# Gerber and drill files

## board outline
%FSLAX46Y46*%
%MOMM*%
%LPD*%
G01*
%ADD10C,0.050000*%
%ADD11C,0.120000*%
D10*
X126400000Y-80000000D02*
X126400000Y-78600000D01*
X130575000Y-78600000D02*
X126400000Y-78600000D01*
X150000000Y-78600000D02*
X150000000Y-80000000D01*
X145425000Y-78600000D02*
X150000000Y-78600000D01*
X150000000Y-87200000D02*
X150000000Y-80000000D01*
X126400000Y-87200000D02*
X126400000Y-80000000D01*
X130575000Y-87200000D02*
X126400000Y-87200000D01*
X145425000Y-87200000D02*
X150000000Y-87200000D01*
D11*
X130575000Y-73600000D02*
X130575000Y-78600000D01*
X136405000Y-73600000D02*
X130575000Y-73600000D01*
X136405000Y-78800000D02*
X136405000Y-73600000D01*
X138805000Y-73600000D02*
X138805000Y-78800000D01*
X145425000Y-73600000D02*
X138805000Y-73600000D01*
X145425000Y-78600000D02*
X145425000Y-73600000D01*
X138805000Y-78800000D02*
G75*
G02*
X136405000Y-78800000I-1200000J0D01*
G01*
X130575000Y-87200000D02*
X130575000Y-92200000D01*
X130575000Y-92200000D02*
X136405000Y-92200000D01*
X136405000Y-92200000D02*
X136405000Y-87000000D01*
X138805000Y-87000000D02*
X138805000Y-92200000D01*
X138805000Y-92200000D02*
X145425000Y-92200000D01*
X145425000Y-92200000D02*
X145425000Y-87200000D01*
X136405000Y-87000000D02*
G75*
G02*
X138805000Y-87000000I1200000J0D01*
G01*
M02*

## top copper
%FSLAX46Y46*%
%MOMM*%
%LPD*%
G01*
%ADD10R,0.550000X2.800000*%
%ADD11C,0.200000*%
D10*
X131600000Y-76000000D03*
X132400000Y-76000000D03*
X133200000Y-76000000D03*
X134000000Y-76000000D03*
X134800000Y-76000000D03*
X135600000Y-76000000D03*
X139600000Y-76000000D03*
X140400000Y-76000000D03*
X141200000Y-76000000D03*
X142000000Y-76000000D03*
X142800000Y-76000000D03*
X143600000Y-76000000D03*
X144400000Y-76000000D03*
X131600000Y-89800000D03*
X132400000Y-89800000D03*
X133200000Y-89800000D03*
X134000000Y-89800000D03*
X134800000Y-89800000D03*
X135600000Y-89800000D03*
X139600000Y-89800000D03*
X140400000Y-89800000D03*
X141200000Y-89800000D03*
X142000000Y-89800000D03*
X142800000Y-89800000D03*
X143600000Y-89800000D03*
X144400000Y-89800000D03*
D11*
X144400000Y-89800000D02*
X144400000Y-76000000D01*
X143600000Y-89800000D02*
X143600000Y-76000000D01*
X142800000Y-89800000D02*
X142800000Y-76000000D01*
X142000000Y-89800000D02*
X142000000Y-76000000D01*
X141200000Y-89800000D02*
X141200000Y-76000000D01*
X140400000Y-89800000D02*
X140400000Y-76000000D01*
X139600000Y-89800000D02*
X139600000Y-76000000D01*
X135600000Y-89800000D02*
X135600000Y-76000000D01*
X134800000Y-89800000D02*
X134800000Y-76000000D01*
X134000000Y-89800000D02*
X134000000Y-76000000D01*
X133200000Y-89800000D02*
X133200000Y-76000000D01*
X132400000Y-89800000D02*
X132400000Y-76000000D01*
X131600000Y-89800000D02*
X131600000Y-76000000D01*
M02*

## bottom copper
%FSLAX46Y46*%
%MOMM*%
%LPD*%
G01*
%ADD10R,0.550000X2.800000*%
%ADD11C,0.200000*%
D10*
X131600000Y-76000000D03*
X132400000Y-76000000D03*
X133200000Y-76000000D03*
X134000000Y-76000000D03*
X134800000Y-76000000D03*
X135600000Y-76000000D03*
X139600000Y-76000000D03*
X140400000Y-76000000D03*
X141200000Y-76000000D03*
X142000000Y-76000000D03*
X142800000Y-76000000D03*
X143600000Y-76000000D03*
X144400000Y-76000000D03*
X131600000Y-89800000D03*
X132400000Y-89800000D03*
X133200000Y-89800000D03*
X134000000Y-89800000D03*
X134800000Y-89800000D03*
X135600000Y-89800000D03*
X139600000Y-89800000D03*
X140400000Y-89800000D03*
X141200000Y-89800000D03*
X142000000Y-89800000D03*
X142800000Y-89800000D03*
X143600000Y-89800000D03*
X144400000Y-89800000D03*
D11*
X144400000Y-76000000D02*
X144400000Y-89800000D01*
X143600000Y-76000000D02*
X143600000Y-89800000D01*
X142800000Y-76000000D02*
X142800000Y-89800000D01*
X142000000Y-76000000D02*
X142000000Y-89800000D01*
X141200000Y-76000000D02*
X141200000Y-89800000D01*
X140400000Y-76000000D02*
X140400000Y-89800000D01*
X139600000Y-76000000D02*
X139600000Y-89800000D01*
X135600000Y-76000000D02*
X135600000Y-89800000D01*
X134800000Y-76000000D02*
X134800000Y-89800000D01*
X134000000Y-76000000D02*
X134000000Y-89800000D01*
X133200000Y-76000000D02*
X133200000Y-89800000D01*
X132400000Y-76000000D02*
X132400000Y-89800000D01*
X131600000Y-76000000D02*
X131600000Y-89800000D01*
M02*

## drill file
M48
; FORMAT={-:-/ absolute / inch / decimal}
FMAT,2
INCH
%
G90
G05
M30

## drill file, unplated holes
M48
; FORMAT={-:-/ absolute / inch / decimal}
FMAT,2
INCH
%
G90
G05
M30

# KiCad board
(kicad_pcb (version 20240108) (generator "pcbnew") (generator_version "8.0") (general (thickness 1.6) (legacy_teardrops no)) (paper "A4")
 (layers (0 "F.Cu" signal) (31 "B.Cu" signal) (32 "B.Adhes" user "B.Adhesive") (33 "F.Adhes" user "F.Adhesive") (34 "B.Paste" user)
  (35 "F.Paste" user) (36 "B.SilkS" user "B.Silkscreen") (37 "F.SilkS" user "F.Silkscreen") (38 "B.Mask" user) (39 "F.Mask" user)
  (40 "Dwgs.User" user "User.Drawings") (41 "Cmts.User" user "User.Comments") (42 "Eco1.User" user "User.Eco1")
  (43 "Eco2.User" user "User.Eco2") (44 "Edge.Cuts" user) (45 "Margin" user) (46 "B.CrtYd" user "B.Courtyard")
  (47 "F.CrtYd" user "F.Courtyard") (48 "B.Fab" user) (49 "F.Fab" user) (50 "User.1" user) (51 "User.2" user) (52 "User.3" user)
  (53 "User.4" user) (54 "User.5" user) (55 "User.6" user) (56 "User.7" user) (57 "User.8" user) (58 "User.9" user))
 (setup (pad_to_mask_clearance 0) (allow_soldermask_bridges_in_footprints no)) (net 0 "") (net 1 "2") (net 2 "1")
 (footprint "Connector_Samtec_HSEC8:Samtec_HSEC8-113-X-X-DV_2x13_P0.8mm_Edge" (layer "F.Cu") (at 138 92.2)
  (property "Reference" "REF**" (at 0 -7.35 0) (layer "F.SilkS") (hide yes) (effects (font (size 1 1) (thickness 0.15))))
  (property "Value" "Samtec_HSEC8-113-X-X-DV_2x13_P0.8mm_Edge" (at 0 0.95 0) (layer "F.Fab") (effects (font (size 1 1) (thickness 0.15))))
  (fp_line (start -7.425 -5) (end -7.425 0) (stroke (width 0.12) (type solid)) (layer "Edge.Cuts"))
  (fp_line (start -7.425 0) (end -1.595 0) (stroke (width 0.12) (type solid)) (layer "Edge.Cuts"))
  (fp_line (start -1.595 0) (end -1.595 -5.2) (stroke (width 0.12) (type solid)) (layer "Edge.Cuts"))
  (fp_line (start 0.805 -5.2) (end 0.805 0) (stroke (width 0.12) (type solid)) (layer "Edge.Cuts"))
  (fp_line (start 0.805 0) (end 7.425 0) (stroke (width 0.12) (type solid)) (layer "Edge.Cuts"))
  (fp_line (start 7.425 0) (end 7.425 -5) (stroke (width 0.12) (type solid)) (layer "Edge.Cuts"))
  (fp_arc (start -1.595 -5.2) (mid -0.395 -6.4) (end 0.805 -5.2) (stroke (width 0.12) (type solid)) (layer "Edge.Cuts"))
  (pad "1" connect rect (at -6.4 -2.4) (size 0.55 2.8) (layers "F.Cu" "F.Mask") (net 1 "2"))
  (pad "2" connect rect (at -6.4 -2.4) (size 0.55 2.8) (layers "B.Cu" "B.Mask") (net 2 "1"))
  (pad "3" connect rect (at -5.6 -2.4) (size 0.55 2.8) (layers "F.Cu" "F.Mask"))
  (pad "4" connect rect (at -5.6 -2.4) (size 0.55 2.8) (layers "B.Cu" "B.Mask"))
  (pad "5" connect rect (at -4.8 -2.4) (size 0.55 2.8) (layers "F.Cu" "F.Mask"))
  (pad "6" connect rect (at -4.8 -2.4) (size 0.55 2.8) (layers "B.Cu" "B.Mask"))
  (pad "7" connect rect (at -4 -2.4) (size 0.55 2.8) (layers "F.Cu" "F.Mask"))
  (pad "8" connect rect (at -4 -2.4) (size 0.55 2.8) (layers "B.Cu" "B.Mask"))
  (pad "9" connect rect (at -3.2 -2.4) (size 0.55 2.8) (layers "F.Cu" "F.Mask"))
  (pad "10" connect rect (at -3.2 -2.4) (size 0.55 2.8) (layers "B.Cu" "B.Mask"))
  (pad "11" connect rect (at -2.4 -2.4) (size 0.55 2.8) (layers "F.Cu" "F.Mask"))
  (pad "12" connect rect (at -2.4 -2.4) (size 0.55 2.8) (layers "B.Cu" "B.Mask"))
  (pad "13" connect rect (at 1.6 -2.4) (size 0.55 2.8) (layers "F.Cu" "F.Mask"))
  (pad "14" connect rect (at 1.6 -2.4) (size 0.55 2.8) (layers "B.Cu" "B.Mask"))
  (pad "15" connect rect (at 2.4 -2.4) (size 0.55 2.8) (layers "F.Cu" "F.Mask"))
  (pad "16" connect rect (at 2.4 -2.4) (size 0.55 2.8) (layers "B.Cu" "B.Mask"))
  (pad "17" connect rect (at 3.2 -2.4) (size 0.55 2.8) (layers "F.Cu" "F.Mask"))
  (pad "18" connect rect (at 3.2 -2.4) (size 0.55 2.8) (layers "B.Cu" "B.Mask"))
  (pad "19" connect rect (at 4 -2.4) (size 0.55 2.8) (layers "F.Cu" "F.Mask"))
  (pad "20" connect rect (at 4 -2.4) (size 0.55 2.8) (layers "B.Cu" "B.Mask"))
  (pad "21" connect rect (at 4.8 -2.4) (size 0.55 2.8) (layers "F.Cu" "F.Mask"))
  (pad "22" connect rect (at 4.8 -2.4) (size 0.55 2.8) (layers "B.Cu" "B.Mask"))
  (pad "23" connect rect (at 5.6 -2.4) (size 0.55 2.8) (layers "F.Cu" "F.Mask"))
  (pad "24" connect rect (at 5.6 -2.4) (size 0.55 2.8) (layers "B.Cu" "B.Mask"))
  (pad "25" connect rect (at 6.4 -2.4) (size 0.55 2.8) (layers "F.Cu" "F.Mask"))
  (pad "26" connect rect (at 6.4 -2.4) (size 0.55 2.8) (layers "B.Cu" "B.Mask")))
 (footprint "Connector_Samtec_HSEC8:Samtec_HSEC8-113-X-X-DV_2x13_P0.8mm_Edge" (layer "B.Cu") (at 138 73.6)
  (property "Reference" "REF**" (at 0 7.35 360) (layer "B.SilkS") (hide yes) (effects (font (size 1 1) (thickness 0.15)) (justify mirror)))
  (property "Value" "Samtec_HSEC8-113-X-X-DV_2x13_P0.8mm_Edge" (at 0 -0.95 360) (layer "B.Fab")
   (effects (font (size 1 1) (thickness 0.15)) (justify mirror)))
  (fp_line (start -7.425 0) (end -7.425 5) (stroke (width 0.12) (type solid)) (layer "Edge.Cuts"))
  (fp_line (start -1.595 0) (end -7.425 0) (stroke (width 0.12) (type solid)) (layer "Edge.Cuts"))
  (fp_line (start -1.595 5.2) (end -1.595 0) (stroke (width 0.12) (type solid)) (layer "Edge.Cuts"))
  (fp_line (start 0.805 0) (end 0.805 5.2) (stroke (width 0.12) (type solid)) (layer "Edge.Cuts"))
  (fp_line (start 7.425 0) (end 0.805 0) (stroke (width 0.12) (type solid)) (layer "Edge.Cuts"))
  (fp_line (start 7.425 5) (end 7.425 0) (stroke (width 0.12) (type solid)) (layer "Edge.Cuts"))
  (fp_arc (start 0.805 5.2) (mid -0.395 6.4) (end -1.595 5.2) (stroke (width 0.12) (type solid)) (layer "Edge.Cuts"))
  (pad "1" connect rect (at -6.4 2.4) (size 0.55 2.8) (layers "B.Cu" "B.Mask") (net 2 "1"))
  (pad "2" connect rect (at -6.4 2.4) (size 0.55 2.8) (layers "F.Cu" "F.Mask") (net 1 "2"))
  (pad "3" connect rect (at -5.6 2.4) (size 0.55 2.8) (layers "B.Cu" "B.Mask"))
  (pad "4" connect rect (at -5.6 2.4) (size 0.55 2.8) (layers "F.Cu" "F.Mask"))
  (pad "5" connect rect (at -4.8 2.4) (size 0.55 2.8) (layers "B.Cu" "B.Mask"))
  (pad "6" connect rect (at -4.8 2.4) (size 0.55 2.8) (layers "F.Cu" "F.Mask"))
  (pad "7" connect rect (at -4 2.4) (size 0.55 2.8) (layers "B.Cu" "B.Mask"))
  (pad "8" connect rect (at -4 2.4) (size 0.55 2.8) (layers "F.Cu" "F.Mask"))
  (pad "9" connect rect (at -3.2 2.4) (size 0.55 2.8) (layers "B.Cu" "B.Mask"))
  (pad "10" connect rect (at -3.2 2.4) (size 0.55 2.8) (layers "F.Cu" "F.Mask"))
  (pad "11" connect rect (at -2.4 2.4) (size 0.55 2.8) (layers "B.Cu" "B.Mask"))
  (pad "12" connect rect (at -2.4 2.4) (size 0.55 2.8) (layers "F.Cu" "F.Mask"))
  (pad "13" connect rect (at 1.6 2.4) (size 0.55 2.8) (layers "B.Cu" "B.Mask"))
  (pad "14" connect rect (at 1.6 2.4) (size 0.55 2.8) (layers "F.Cu" "F.Mask"))
  (pad "15" connect rect (at 2.4 2.4) (size 0.55 2.8) (layers "B.Cu" "B.Mask"))
  (pad "16" connect rect (at 2.4 2.4) (size 0.55 2.8) (layers "F.Cu" "F.Mask"))
  (pad "17" connect rect (at 3.2 2.4) (size 0.55 2.8) (layers "B.Cu" "B.Mask"))
  (pad "18" connect rect (at 3.2 2.4) (size 0.55 2.8) (layers "F.Cu" "F.Mask"))
  (pad "19" connect rect (at 4 2.4) (size 0.55 2.8) (layers "B.Cu" "B.Mask"))
  (pad "20" connect rect (at 4 2.4) (size 0.55 2.8) (layers "F.Cu" "F.Mask"))
  (pad "21" connect rect (at 4.8 2.4) (size 0.55 2.8) (layers "B.Cu" "B.Mask"))
  (pad "22" connect rect (at 4.8 2.4) (size 0.55 2.8) (layers "F.Cu" "F.Mask"))
  (pad "23" connect rect (at 5.6 2.4) (size 0.55 2.8) (layers "B.Cu" "B.Mask"))
  (pad "24" connect rect (at 5.6 2.4) (size 0.55 2.8) (layers "F.Cu" "F.Mask"))
  (pad "25" connect rect (at 6.4 2.4) (size 0.55 2.8) (layers "B.Cu" "B.Mask"))
  (pad "26" connect rect (at 6.4 2.4) (size 0.55 2.8) (layers "F.Cu" "F.Mask")))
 (gr_line (start 130.575 78.6) (end 126.4 78.6) (stroke (width 0.05) (type default)) (layer "Edge.Cuts"))
 (gr_line (start 150 87.2) (end 150 80) (stroke (width 0.05) (type default)) (layer "Edge.Cuts"))
 (gr_line (start 126.4 87.2) (end 126.4 80) (stroke (width 0.05) (type default)) (layer "Edge.Cuts"))
 (gr_line (start 130.575 87.2) (end 126.4 87.2) (stroke (width 0.05) (type default)) (layer "Edge.Cuts"))
 (gr_line (start 150 78.6) (end 150 80) (stroke (width 0.05) (type default)) (layer "Edge.Cuts"))
 (gr_line (start 126.4 80) (end 126.4 78.6) (stroke (width 0.05) (type default)) (layer "Edge.Cuts"))
 (gr_line (start 145.425 87.2) (end 150 87.2) (stroke (width 0.05) (type default)) (layer "Edge.Cuts"))
 (gr_line (start 145.425 78.6) (end 150 78.6) (stroke (width 0.05) (type default)) (layer "Edge.Cuts"))
 (segment (start 141.2 89.8) (end 141.2 76) (width 0.2) (layer "F.Cu") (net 1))
 (segment (start 140.4 89.8) (end 140.4 76) (width 0.2) (layer "F.Cu") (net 1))
 (segment (start 131.6 89.8) (end 131.6 76) (width 0.2) (layer "F.Cu") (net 1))
 (segment (start 144.4 89.8) (end 144.4 76) (width 0.2) (layer "F.Cu") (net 1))
 (segment (start 142 89.8) (end 142 76) (width 0.2) (layer "F.Cu") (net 1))
 (segment (start 132.4 89.8) (end 132.4 76) (width 0.2) (layer "F.Cu") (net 1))
 (segment (start 139.6 89.8) (end 139.6 76) (width 0.2) (layer "F.Cu") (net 1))
 (segment (start 142.8 89.8) (end 142.8 76) (width 0.2) (layer "F.Cu") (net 1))
 (segment (start 143.6 89.8) (end 143.6 76) (width 0.2) (layer "F.Cu") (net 1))
 (segment (start 134.8 89.8) (end 134.8 76) (width 0.2) (layer "F.Cu") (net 1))
 (segment (start 134 89.8) (end 134 76) (width 0.2) (layer "F.Cu") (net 1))
 (segment (start 133.2 89.8) (end 133.2 76) (width 0.2) (layer "F.Cu") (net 1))
 (segment (start 135.6 89.8) (end 135.6 76) (width 0.2) (layer "F.Cu") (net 1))
 (segment (start 142 76) (end 142 89.8) (width 0.2) (layer "B.Cu") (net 2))
 (segment (start 131.6 76) (end 131.6 89.8) (width 0.2) (layer "B.Cu") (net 2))
 (segment (start 144.4 76) (end 144.4 89.8) (width 0.2) (layer "B.Cu") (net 2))
 (segment (start 141.2 76) (end 141.2 89.8) (width 0.2) (layer "B.Cu") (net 2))
 (segment (start 139.6 76) (end 139.6 89.8) (width 0.2) (layer "B.Cu") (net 2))
 (segment (start 142.8 76) (end 142.8 89.8) (width 0.2) (layer "B.Cu") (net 2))
 (segment (start 134 76) (end 134 89.8) (width 0.2) (layer "B.Cu") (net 2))
 (segment (start 140.4 76) (end 140.4 89.8) (width 0.2) (layer "B.Cu") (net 2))
 (segment (start 143.6 76) (end 143.6 89.8) (width 0.2) (layer "B.Cu") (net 2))
 (segment (start 132.4 76) (end 132.4 89.8) (width 0.2) (layer "B.Cu") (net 2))
 (segment (start 135.6 76) (end 135.6 89.8) (width 0.2) (layer "B.Cu") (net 2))
 (segment (start 133.2 76) (end 133.2 89.8) (width 0.2) (layer "B.Cu") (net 2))
 (segment (start 134.8 76) (end 134.8 89.8) (width 0.2) (layer "B.Cu") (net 2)))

